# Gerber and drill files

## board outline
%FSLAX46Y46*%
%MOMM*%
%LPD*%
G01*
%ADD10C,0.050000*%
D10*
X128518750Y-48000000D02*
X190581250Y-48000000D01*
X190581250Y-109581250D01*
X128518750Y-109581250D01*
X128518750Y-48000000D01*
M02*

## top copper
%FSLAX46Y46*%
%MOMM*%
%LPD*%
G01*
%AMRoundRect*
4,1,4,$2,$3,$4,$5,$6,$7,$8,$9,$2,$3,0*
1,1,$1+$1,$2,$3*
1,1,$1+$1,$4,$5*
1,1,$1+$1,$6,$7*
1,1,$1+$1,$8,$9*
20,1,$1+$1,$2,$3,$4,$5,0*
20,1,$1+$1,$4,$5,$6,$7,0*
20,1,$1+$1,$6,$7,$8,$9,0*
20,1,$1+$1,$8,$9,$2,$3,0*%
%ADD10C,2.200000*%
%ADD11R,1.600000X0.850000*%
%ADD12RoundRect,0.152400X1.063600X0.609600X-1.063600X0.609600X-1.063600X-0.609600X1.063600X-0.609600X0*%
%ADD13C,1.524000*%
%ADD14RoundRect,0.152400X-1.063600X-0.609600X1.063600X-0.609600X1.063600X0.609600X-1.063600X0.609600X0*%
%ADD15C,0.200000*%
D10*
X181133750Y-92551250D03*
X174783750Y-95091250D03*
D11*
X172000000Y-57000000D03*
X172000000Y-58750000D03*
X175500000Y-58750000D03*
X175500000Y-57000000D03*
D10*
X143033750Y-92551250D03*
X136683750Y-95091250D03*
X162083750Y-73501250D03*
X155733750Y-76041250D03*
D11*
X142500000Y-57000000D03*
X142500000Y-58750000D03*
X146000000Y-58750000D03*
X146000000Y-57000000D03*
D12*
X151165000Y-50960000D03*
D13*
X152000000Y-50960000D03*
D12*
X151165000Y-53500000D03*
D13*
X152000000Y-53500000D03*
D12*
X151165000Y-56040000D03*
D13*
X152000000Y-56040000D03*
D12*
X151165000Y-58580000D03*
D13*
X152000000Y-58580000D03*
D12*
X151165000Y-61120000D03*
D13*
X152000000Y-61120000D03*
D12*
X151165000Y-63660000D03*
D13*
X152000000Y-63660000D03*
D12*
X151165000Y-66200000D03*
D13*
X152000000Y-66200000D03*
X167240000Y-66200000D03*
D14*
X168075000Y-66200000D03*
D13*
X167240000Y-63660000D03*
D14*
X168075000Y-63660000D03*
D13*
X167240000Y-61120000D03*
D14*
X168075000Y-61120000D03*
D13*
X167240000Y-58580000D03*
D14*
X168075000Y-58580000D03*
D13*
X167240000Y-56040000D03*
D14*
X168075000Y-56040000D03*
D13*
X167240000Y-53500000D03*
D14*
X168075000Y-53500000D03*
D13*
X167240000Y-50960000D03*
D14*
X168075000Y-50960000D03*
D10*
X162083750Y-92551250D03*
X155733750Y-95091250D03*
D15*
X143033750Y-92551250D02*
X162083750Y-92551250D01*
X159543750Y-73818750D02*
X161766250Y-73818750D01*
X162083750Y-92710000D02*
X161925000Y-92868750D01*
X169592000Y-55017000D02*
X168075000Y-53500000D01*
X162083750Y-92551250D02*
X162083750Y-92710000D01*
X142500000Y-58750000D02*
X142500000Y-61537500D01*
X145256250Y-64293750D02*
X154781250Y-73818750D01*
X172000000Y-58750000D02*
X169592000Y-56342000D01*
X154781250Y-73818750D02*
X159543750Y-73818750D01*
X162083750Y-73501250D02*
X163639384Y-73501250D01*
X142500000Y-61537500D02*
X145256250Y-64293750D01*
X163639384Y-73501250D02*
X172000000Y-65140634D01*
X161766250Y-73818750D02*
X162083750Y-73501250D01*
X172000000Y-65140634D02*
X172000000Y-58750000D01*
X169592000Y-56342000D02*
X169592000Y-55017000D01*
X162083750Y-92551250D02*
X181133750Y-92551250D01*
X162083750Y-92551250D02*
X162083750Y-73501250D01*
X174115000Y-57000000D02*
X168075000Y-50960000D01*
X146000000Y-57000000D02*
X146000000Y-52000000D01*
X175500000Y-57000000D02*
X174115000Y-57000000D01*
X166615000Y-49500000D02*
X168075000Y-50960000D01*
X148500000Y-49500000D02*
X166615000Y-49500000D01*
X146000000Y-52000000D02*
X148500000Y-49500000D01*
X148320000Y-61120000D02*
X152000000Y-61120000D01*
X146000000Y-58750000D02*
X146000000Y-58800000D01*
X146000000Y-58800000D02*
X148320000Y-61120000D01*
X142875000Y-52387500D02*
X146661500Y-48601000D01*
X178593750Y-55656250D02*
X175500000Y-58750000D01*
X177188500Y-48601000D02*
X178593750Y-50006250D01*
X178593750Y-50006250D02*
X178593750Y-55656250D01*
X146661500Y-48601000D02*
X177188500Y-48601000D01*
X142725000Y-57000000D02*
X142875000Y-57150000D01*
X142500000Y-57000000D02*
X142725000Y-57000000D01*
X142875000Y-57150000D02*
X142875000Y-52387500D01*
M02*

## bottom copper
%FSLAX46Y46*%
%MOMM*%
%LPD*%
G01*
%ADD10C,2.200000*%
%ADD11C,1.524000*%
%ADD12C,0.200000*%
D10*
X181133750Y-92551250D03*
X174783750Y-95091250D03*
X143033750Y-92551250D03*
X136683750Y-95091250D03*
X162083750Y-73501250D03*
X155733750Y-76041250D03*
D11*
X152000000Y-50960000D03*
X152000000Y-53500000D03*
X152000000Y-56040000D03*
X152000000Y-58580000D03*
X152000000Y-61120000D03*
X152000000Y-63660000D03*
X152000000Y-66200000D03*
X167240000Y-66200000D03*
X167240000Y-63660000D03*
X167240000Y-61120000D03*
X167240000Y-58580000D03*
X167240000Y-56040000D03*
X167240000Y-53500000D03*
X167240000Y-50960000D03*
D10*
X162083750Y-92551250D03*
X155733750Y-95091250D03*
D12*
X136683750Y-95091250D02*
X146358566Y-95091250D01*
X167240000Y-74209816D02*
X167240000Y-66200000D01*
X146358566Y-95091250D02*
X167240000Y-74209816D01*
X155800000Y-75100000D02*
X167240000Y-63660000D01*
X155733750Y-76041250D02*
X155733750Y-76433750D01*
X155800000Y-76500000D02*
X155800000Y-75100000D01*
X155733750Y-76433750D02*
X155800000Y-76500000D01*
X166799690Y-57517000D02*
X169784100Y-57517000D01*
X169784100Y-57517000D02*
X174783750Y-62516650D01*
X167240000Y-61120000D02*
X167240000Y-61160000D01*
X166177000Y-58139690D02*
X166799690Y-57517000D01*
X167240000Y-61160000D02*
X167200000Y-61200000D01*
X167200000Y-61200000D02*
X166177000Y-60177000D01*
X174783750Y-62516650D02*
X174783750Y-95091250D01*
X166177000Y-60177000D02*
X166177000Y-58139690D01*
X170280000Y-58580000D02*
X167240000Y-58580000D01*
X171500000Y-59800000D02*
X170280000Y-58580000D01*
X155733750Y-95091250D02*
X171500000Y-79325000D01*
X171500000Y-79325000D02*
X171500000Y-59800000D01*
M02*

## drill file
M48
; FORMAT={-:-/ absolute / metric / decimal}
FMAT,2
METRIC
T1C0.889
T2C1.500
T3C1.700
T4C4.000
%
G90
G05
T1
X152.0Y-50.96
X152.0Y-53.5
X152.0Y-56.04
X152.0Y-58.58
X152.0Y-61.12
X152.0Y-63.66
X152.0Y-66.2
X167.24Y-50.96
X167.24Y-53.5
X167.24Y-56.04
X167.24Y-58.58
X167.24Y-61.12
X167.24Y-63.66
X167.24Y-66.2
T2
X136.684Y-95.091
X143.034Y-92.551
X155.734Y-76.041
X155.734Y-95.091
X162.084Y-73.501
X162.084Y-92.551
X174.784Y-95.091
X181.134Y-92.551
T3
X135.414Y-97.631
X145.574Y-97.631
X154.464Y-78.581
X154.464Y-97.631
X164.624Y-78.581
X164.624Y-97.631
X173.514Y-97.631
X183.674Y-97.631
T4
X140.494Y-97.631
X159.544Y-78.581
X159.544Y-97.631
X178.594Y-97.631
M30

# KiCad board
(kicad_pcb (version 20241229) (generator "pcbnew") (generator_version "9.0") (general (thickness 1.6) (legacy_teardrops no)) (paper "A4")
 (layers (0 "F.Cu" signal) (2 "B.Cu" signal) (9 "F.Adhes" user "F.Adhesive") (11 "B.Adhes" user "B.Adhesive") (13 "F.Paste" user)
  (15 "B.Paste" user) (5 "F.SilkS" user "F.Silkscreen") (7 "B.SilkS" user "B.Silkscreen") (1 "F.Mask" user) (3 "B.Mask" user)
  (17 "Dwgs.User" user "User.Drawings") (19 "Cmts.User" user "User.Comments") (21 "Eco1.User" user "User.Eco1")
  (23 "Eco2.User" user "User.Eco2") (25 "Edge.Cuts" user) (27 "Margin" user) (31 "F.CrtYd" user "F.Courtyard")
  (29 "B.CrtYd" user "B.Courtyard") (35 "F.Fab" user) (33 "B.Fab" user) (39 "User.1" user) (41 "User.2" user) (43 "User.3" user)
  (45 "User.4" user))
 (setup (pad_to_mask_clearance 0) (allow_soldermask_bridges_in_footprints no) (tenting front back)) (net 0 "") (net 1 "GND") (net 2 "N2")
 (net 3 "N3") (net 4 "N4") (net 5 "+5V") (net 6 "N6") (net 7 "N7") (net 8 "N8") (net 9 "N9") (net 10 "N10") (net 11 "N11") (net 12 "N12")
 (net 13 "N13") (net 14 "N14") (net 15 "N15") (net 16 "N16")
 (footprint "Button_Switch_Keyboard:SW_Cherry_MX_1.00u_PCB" (layer "F.Cu") (at 181.13375 92.55125)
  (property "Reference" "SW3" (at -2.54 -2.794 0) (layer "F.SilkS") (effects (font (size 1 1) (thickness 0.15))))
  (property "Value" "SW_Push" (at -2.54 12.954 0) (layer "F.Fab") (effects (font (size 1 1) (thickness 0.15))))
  (pad "" np_thru_hole circle (at -7.62 5.08) (size 1.7 1.7) (drill 1.7) (layers "*.Cu" "*.Mask"))
  (pad "" np_thru_hole circle (at -2.54 5.08) (size 4 4) (drill 4) (layers "*.Cu" "*.Mask"))
  (pad "" np_thru_hole circle (at 2.54 5.08) (size 1.7 1.7) (drill 1.7) (layers "*.Cu" "*.Mask"))
  (pad "1" thru_hole circle (at 0 0) (size 2.2 2.2) (drill 1.5) (layers "*.Cu" "*.Mask") (remove_unused_layers no) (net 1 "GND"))
  (pad "2" thru_hole circle (at -6.35 2.54) (size 2.2 2.2) (drill 1.5) (layers "*.Cu" "*.Mask") (remove_unused_layers no) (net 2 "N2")))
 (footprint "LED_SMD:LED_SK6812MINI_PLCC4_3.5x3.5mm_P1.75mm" (layer "F.Cu") (at 173.75 57.875)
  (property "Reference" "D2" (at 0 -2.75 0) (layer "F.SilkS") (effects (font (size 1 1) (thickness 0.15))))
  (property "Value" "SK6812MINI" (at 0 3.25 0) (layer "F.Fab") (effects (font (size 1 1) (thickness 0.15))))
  (pad "1" smd rect (at -1.75 -0.875) (size 1.6 0.85) (layers "F.Cu" "F.Mask" "F.Paste") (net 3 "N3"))
  (pad "2" smd rect (at -1.75 0.875) (size 1.6 0.85) (layers "F.Cu" "F.Mask" "F.Paste") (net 1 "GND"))
  (pad "3" smd rect (at 1.75 0.875) (size 1.6 0.85) (layers "F.Cu" "F.Mask" "F.Paste") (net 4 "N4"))
  (pad "4" smd rect (at 1.75 -0.875) (size 1.6 0.85) (layers "F.Cu" "F.Mask" "F.Paste") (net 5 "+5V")))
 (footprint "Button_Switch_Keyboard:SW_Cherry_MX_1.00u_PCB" (layer "F.Cu") (at 143.03375 92.55125)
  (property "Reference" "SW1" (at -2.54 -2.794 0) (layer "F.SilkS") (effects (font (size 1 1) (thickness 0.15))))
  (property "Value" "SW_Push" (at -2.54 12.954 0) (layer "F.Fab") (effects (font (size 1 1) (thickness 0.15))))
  (pad "" np_thru_hole circle (at -7.62 5.08) (size 1.7 1.7) (drill 1.7) (layers "*.Cu" "*.Mask"))
  (pad "" np_thru_hole circle (at -2.54 5.08) (size 4 4) (drill 4) (layers "*.Cu" "*.Mask"))
  (pad "" np_thru_hole circle (at 2.54 5.08) (size 1.7 1.7) (drill 1.7) (layers "*.Cu" "*.Mask"))
  (pad "1" thru_hole circle (at 0 0) (size 2.2 2.2) (drill 1.5) (layers "*.Cu" "*.Mask") (remove_unused_layers no) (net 1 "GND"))
  (pad "2" thru_hole circle (at -6.35 2.54) (size 2.2 2.2) (drill 1.5) (layers "*.Cu" "*.Mask") (remove_unused_layers no) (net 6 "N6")))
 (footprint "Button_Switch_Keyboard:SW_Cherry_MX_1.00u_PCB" (layer "F.Cu") (at 162.08375 73.50125)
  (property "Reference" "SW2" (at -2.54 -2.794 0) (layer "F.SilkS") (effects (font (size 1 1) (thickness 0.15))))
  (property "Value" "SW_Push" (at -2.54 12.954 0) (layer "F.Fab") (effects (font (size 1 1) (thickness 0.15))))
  (pad "" np_thru_hole circle (at -7.62 5.08) (size 1.7 1.7) (drill 1.7) (layers "*.Cu" "*.Mask"))
  (pad "" np_thru_hole circle (at -2.54 5.08) (size 4 4) (drill 4) (layers "*.Cu" "*.Mask"))
  (pad "" np_thru_hole circle (at 2.54 5.08) (size 1.7 1.7) (drill 1.7) (layers "*.Cu" "*.Mask"))
  (pad "1" thru_hole circle (at 0 0) (size 2.2 2.2) (drill 1.5) (layers "*.Cu" "*.Mask") (remove_unused_layers no) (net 1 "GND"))
  (pad "2" thru_hole circle (at -6.35 2.54) (size 2.2 2.2) (drill 1.5) (layers "*.Cu" "*.Mask") (remove_unused_layers no) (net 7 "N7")))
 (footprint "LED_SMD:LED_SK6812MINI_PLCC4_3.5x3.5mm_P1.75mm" (layer "F.Cu") (at 144.25 57.875)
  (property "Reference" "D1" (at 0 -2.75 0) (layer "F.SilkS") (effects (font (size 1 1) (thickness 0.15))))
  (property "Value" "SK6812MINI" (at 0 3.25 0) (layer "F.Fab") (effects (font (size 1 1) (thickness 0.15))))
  (pad "1" smd rect (at -1.75 -0.875) (size 1.6 0.85) (layers "F.Cu" "F.Mask" "F.Paste") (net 4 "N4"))
  (pad "2" smd rect (at -1.75 0.875) (size 1.6 0.85) (layers "F.Cu" "F.Mask" "F.Paste") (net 1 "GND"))
  (pad "3" smd rect (at 1.75 0.875) (size 1.6 0.85) (layers "F.Cu" "F.Mask" "F.Paste") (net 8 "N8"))
  (pad "4" smd rect (at 1.75 -0.875) (size 1.6 0.85) (layers "F.Cu" "F.Mask" "F.Paste") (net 5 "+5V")))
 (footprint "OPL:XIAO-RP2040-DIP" (layer "F.Cu") (at 159.62 58.58)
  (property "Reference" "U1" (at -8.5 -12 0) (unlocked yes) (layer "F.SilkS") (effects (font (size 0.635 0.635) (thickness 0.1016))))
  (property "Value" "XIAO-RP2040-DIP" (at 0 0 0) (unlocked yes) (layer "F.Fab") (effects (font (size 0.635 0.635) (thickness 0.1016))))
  (pad "1" smd roundrect (at -8.455 -7.62 180) (size 2.432 1.524) (layers "F.Cu" "F.Mask") (roundrect_rratio 0.1) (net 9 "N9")
   (thermal_bridge_angle 45))
  (pad "1" thru_hole circle (at -7.62 -7.62 180) (size 1.524 1.524) (drill 0.889) (layers "*.Cu" "*.Mask") (remove_unused_layers no)
   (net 9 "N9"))
  (pad "2" smd roundrect (at -8.455 -5.08 180) (size 2.432 1.524) (layers "F.Cu" "F.Mask") (roundrect_rratio 0.1) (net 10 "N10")
   (thermal_bridge_angle 45))
  (pad "2" thru_hole circle (at -7.62 -5.08 180) (size 1.524 1.524) (drill 0.889) (layers "*.Cu" "*.Mask") (remove_unused_layers no)
   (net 10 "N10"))
  (pad "3" smd roundrect (at -8.455 -2.54 180) (size 2.432 1.524) (layers "F.Cu" "F.Mask") (roundrect_rratio 0.1) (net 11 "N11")
   (thermal_bridge_angle 45))
  (pad "3" thru_hole circle (at -7.62 -2.54 180) (size 1.524 1.524) (drill 0.889) (layers "*.Cu" "*.Mask") (remove_unused_layers no)
   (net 11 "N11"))
  (pad "4" smd roundrect (at -8.455 0 180) (size 2.432 1.524) (layers "F.Cu" "F.Mask") (roundrect_rratio 0.1) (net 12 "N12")
   (thermal_bridge_angle 45))
  (pad "4" thru_hole circle (at -7.62 0 180) (size 1.524 1.524) (drill 0.889) (layers "*.Cu" "*.Mask") (remove_unused_layers no)
   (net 12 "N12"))
  (pad "5" smd roundrect (at -8.455 2.54 180) (size 2.432 1.524) (layers "F.Cu" "F.Mask") (roundrect_rratio 0.1) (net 8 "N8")
   (thermal_bridge_angle 45))
  (pad "5" thru_hole circle (at -7.62 2.54 180) (size 1.524 1.524) (drill 0.889) (layers "*.Cu" "*.Mask") (remove_unused_layers no)
   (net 8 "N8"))
  (pad "6" smd roundrect (at -8.455 5.08 180) (size 2.432 1.524) (layers "F.Cu" "F.Mask") (roundrect_rratio 0.1) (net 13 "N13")
   (thermal_bridge_angle 45))
  (pad "6" thru_hole circle (at -7.62 5.08 180) (size 1.524 1.524) (drill 0.889) (layers "*.Cu" "*.Mask") (remove_unused_layers no)
   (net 13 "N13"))
  (pad "7" smd roundrect (at -8.455 7.62 180) (size 2.432 1.524) (layers "F.Cu" "F.Mask") (roundrect_rratio 0.1) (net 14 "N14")
   (thermal_bridge_angle 45))
  (pad "7" thru_hole circle (at -7.62 7.62 180) (size 1.524 1.524) (drill 0.889) (layers "*.Cu" "*.Mask") (remove_unused_layers no)
   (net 14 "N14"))
  (pad "8" thru_hole circle (at 7.62 7.62) (size 1.524 1.524) (drill 0.889) (layers "*.Cu" "*.Mask") (remove_unused_layers no) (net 6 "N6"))
  (pad "8" smd roundrect (at 8.455 7.62) (size 2.432 1.524) (layers "F.Cu" "F.Mask") (roundrect_rratio 0.1) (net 6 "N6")
   (thermal_bridge_angle 45))
  (pad "9" thru_hole circle (at 7.62 5.08) (size 1.524 1.524) (drill 0.889) (layers "*.Cu" "*.Mask") (remove_unused_layers no) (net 7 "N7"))
  (pad "9" smd roundrect (at 8.455 5.08) (size 2.432 1.524) (layers "F.Cu" "F.Mask") (roundrect_rratio 0.1) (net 7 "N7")
   (thermal_bridge_angle 45))
  (pad "10" thru_hole circle (at 7.62 2.54) (size 1.524 1.524) (drill 0.889) (layers "*.Cu" "*.Mask") (remove_unused_layers no) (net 2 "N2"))
  (pad "10" smd roundrect (at 8.455 2.54) (size 2.432 1.524) (layers "F.Cu" "F.Mask") (roundrect_rratio 0.1) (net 2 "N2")
   (thermal_bridge_angle 45))
  (pad "11" thru_hole circle (at 7.62 0) (size 1.524 1.524) (drill 0.889) (layers "*.Cu" "*.Mask") (remove_unused_layers no) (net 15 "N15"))
  (pad "11" smd roundrect (at 8.455 0) (size 2.432 1.524) (layers "F.Cu" "F.Mask") (roundrect_rratio 0.1) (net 15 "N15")
   (thermal_bridge_angle 45))
  (pad "12" thru_hole circle (at 7.62 -2.54) (size 1.524 1.524) (drill 0.889) (layers "*.Cu" "*.Mask") (remove_unused_layers no)
   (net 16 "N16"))
  (pad "12" smd roundrect (at 8.455 -2.54) (size 2.432 1.524) (layers "F.Cu" "F.Mask") (roundrect_rratio 0.1) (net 16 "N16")
   (thermal_bridge_angle 45))
  (pad "13" thru_hole circle (at 7.62 -5.08) (size 1.524 1.524) (drill 0.889) (layers "*.Cu" "*.Mask") (remove_unused_layers no)
   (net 1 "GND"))
  (pad "13" smd roundrect (at 8.455 -5.08) (size 2.432 1.524) (layers "F.Cu" "F.Mask") (roundrect_rratio 0.1) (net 1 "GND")
   (thermal_bridge_angle 45))
  (pad "14" thru_hole circle (at 7.62 -7.62) (size 1.524 1.524) (drill 0.889) (layers "*.Cu" "*.Mask") (remove_unused_layers no)
   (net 5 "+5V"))
  (pad "14" smd roundrect (at 8.455 -7.62) (size 2.432 1.524) (layers "F.Cu" "F.Mask") (roundrect_rratio 0.1) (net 5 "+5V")
   (thermal_bridge_angle 45)))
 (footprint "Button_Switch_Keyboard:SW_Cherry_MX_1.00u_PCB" (layer "F.Cu") (at 162.08375 92.55125)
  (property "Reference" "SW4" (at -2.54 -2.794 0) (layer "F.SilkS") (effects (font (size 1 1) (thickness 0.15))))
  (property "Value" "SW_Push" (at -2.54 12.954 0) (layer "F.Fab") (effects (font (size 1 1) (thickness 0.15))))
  (pad "" np_thru_hole circle (at -7.62 5.08) (size 1.7 1.7) (drill 1.7) (layers "*.Cu" "*.Mask"))
  (pad "" np_thru_hole circle (at -2.54 5.08) (size 4 4) (drill 4) (layers "*.Cu" "*.Mask"))
  (pad "" np_thru_hole circle (at 2.54 5.08) (size 1.7 1.7) (drill 1.7) (layers "*.Cu" "*.Mask"))
  (pad "1" thru_hole circle (at 0 0) (size 2.2 2.2) (drill 1.5) (layers "*.Cu" "*.Mask") (remove_unused_layers no) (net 1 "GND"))
  (pad "2" thru_hole circle (at -6.35 2.54) (size 2.2 2.2) (drill 1.5) (layers "*.Cu" "*.Mask") (remove_unused_layers no) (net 15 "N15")))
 (gr_rect (start 128.51875 48) (end 190.58125 109.58125) (stroke (width 0.05) (type default)) (fill no) (layer "Edge.Cuts"))
 (segment (start 143.03375 92.55125) (end 162.08375 92.55125) (width 0.2) (layer "F.Cu") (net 1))
 (segment (start 159.54375 73.81875) (end 161.76625 73.81875) (width 0.2) (layer "F.Cu") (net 1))
 (segment (start 162.08375 92.71) (end 161.925 92.86875) (width 0.2) (layer "F.Cu") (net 1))
 (segment (start 169.592 55.017) (end 168.075 53.5) (width 0.2) (layer "F.Cu") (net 1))
 (segment (start 162.08375 92.55125) (end 162.08375 92.71) (width 0.2) (layer "F.Cu") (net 1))
 (segment (start 142.5 58.75) (end 142.5 61.5375) (width 0.2) (layer "F.Cu") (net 1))
 (segment (start 145.25625 64.29375) (end 154.78125 73.81875) (width 0.2) (layer "F.Cu") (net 1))
 (segment (start 172 58.75) (end 169.592 56.342) (width 0.2) (layer "F.Cu") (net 1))
 (segment (start 154.78125 73.81875) (end 159.54375 73.81875) (width 0.2) (layer "F.Cu") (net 1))
 (segment (start 162.08375 73.50125) (end 163.639384 73.50125) (width 0.2) (layer "F.Cu") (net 1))
 (segment (start 142.5 61.5375) (end 145.25625 64.29375) (width 0.2) (layer "F.Cu") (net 1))
 (segment (start 163.639384 73.50125) (end 172 65.140634) (width 0.2) (layer "F.Cu") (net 1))
 (segment (start 161.76625 73.81875) (end 162.08375 73.50125) (width 0.2) (layer "F.Cu") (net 1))
 (segment (start 172 65.140634) (end 172 58.75) (width 0.2) (layer "F.Cu") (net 1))
 (segment (start 169.592 56.342) (end 169.592 55.017) (width 0.2) (layer "F.Cu") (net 1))
 (segment (start 162.08375 92.55125) (end 181.13375 92.55125) (width 0.2) (layer "F.Cu") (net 1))
 (segment (start 162.08375 92.55125) (end 162.08375 73.50125) (width 0.2) (layer "F.Cu") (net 1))
 (segment (start 174.115 57) (end 168.075 50.96) (width 0.2) (layer "F.Cu") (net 5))
 (segment (start 146 57) (end 146 52) (width 0.2) (layer "F.Cu") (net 5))
 (segment (start 175.5 57) (end 174.115 57) (width 0.2) (layer "F.Cu") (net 5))
 (segment (start 166.615 49.5) (end 168.075 50.96) (width 0.2) (layer "F.Cu") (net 5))
 (segment (start 148.5 49.5) (end 166.615 49.5) (width 0.2) (layer "F.Cu") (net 5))
 (segment (start 146 52) (end 148.5 49.5) (width 0.2) (layer "F.Cu") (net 5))
 (segment (start 148.32 61.12) (end 152 61.12) (width 0.2) (layer "F.Cu") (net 8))
 (segment (start 146 58.75) (end 146 58.8) (width 0.2) (layer "F.Cu") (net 8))
 (segment (start 146 58.8) (end 148.32 61.12) (width 0.2) (layer "F.Cu") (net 8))
 (segment (start 142.875 52.3875) (end 146.6615 48.601) (width 0.2) (layer "F.Cu") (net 4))
 (segment (start 178.59375 55.65625) (end 175.5 58.75) (width 0.2) (layer "F.Cu") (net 4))
 (segment (start 177.1885 48.601) (end 178.59375 50.00625) (width 0.2) (layer "F.Cu") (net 4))
 (segment (start 178.59375 50.00625) (end 178.59375 55.65625) (width 0.2) (layer "F.Cu") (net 4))
 (segment (start 146.6615 48.601) (end 177.1885 48.601) (width 0.2) (layer "F.Cu") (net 4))
 (segment (start 142.725 57) (end 142.875 57.15) (width 0.2) (layer "F.Cu") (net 4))
 (segment (start 142.5 57) (end 142.725 57) (width 0.2) (layer "F.Cu") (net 4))
 (segment (start 142.875 57.15) (end 142.875 52.3875) (width 0.2) (layer "F.Cu") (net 4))
 (segment (start 136.68375 95.09125) (end 146.358566 95.09125) (width 0.2) (layer "B.Cu") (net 6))
 (segment (start 167.24 74.209816) (end 167.24 66.2) (width 0.2) (layer "B.Cu") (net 6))
 (segment (start 146.358566 95.09125) (end 167.24 74.209816) (width 0.2) (layer "B.Cu") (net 6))
 (segment (start 155.8 75.1) (end 167.24 63.66) (width 0.2) (layer "B.Cu") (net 7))
 (segment (start 155.73375 76.04125) (end 155.73375 76.43375) (width 0.2) (layer "B.Cu") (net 7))
 (segment (start 155.8 76.5) (end 155.8 75.1) (width 0.2) (layer "B.Cu") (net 7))
 (segment (start 155.73375 76.43375) (end 155.8 76.5) (width 0.2) (layer "B.Cu") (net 7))
 (segment (start 166.79969 57.517) (end 169.7841 57.517) (width 0.2) (layer "B.Cu") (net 2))
 (segment (start 169.7841 57.517) (end 174.78375 62.51665) (width 0.2) (layer "B.Cu") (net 2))
 (segment (start 167.24 61.12) (end 167.24 61.16) (width 0.2) (layer "B.Cu") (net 2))
 (segment (start 166.177 58.13969) (end 166.79969 57.517) (width 0.2) (layer "B.Cu") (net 2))
 (segment (start 167.24 61.16) (end 167.2 61.2) (width 0.2) (layer "B.Cu") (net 2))
 (segment (start 167.2 61.2) (end 166.177 60.177) (width 0.2) (layer "B.Cu") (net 2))
 (segment (start 174.78375 62.51665) (end 174.78375 95.09125) (width 0.2) (layer "B.Cu") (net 2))
 (segment (start 166.177 60.177) (end 166.177 58.13969) (width 0.2) (layer "B.Cu") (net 2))
 (segment (start 170.28 58.58) (end 167.24 58.58) (width 0.2) (layer "B.Cu") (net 15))
 (segment (start 171.5 59.8) (end 170.28 58.58) (width 0.2) (layer "B.Cu") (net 15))
 (segment (start 155.73375 95.09125) (end 171.5 79.325) (width 0.2) (layer "B.Cu") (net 15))
 (segment (start 171.5 79.325) (end 171.5 59.8) (width 0.2) (layer "B.Cu") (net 15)))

